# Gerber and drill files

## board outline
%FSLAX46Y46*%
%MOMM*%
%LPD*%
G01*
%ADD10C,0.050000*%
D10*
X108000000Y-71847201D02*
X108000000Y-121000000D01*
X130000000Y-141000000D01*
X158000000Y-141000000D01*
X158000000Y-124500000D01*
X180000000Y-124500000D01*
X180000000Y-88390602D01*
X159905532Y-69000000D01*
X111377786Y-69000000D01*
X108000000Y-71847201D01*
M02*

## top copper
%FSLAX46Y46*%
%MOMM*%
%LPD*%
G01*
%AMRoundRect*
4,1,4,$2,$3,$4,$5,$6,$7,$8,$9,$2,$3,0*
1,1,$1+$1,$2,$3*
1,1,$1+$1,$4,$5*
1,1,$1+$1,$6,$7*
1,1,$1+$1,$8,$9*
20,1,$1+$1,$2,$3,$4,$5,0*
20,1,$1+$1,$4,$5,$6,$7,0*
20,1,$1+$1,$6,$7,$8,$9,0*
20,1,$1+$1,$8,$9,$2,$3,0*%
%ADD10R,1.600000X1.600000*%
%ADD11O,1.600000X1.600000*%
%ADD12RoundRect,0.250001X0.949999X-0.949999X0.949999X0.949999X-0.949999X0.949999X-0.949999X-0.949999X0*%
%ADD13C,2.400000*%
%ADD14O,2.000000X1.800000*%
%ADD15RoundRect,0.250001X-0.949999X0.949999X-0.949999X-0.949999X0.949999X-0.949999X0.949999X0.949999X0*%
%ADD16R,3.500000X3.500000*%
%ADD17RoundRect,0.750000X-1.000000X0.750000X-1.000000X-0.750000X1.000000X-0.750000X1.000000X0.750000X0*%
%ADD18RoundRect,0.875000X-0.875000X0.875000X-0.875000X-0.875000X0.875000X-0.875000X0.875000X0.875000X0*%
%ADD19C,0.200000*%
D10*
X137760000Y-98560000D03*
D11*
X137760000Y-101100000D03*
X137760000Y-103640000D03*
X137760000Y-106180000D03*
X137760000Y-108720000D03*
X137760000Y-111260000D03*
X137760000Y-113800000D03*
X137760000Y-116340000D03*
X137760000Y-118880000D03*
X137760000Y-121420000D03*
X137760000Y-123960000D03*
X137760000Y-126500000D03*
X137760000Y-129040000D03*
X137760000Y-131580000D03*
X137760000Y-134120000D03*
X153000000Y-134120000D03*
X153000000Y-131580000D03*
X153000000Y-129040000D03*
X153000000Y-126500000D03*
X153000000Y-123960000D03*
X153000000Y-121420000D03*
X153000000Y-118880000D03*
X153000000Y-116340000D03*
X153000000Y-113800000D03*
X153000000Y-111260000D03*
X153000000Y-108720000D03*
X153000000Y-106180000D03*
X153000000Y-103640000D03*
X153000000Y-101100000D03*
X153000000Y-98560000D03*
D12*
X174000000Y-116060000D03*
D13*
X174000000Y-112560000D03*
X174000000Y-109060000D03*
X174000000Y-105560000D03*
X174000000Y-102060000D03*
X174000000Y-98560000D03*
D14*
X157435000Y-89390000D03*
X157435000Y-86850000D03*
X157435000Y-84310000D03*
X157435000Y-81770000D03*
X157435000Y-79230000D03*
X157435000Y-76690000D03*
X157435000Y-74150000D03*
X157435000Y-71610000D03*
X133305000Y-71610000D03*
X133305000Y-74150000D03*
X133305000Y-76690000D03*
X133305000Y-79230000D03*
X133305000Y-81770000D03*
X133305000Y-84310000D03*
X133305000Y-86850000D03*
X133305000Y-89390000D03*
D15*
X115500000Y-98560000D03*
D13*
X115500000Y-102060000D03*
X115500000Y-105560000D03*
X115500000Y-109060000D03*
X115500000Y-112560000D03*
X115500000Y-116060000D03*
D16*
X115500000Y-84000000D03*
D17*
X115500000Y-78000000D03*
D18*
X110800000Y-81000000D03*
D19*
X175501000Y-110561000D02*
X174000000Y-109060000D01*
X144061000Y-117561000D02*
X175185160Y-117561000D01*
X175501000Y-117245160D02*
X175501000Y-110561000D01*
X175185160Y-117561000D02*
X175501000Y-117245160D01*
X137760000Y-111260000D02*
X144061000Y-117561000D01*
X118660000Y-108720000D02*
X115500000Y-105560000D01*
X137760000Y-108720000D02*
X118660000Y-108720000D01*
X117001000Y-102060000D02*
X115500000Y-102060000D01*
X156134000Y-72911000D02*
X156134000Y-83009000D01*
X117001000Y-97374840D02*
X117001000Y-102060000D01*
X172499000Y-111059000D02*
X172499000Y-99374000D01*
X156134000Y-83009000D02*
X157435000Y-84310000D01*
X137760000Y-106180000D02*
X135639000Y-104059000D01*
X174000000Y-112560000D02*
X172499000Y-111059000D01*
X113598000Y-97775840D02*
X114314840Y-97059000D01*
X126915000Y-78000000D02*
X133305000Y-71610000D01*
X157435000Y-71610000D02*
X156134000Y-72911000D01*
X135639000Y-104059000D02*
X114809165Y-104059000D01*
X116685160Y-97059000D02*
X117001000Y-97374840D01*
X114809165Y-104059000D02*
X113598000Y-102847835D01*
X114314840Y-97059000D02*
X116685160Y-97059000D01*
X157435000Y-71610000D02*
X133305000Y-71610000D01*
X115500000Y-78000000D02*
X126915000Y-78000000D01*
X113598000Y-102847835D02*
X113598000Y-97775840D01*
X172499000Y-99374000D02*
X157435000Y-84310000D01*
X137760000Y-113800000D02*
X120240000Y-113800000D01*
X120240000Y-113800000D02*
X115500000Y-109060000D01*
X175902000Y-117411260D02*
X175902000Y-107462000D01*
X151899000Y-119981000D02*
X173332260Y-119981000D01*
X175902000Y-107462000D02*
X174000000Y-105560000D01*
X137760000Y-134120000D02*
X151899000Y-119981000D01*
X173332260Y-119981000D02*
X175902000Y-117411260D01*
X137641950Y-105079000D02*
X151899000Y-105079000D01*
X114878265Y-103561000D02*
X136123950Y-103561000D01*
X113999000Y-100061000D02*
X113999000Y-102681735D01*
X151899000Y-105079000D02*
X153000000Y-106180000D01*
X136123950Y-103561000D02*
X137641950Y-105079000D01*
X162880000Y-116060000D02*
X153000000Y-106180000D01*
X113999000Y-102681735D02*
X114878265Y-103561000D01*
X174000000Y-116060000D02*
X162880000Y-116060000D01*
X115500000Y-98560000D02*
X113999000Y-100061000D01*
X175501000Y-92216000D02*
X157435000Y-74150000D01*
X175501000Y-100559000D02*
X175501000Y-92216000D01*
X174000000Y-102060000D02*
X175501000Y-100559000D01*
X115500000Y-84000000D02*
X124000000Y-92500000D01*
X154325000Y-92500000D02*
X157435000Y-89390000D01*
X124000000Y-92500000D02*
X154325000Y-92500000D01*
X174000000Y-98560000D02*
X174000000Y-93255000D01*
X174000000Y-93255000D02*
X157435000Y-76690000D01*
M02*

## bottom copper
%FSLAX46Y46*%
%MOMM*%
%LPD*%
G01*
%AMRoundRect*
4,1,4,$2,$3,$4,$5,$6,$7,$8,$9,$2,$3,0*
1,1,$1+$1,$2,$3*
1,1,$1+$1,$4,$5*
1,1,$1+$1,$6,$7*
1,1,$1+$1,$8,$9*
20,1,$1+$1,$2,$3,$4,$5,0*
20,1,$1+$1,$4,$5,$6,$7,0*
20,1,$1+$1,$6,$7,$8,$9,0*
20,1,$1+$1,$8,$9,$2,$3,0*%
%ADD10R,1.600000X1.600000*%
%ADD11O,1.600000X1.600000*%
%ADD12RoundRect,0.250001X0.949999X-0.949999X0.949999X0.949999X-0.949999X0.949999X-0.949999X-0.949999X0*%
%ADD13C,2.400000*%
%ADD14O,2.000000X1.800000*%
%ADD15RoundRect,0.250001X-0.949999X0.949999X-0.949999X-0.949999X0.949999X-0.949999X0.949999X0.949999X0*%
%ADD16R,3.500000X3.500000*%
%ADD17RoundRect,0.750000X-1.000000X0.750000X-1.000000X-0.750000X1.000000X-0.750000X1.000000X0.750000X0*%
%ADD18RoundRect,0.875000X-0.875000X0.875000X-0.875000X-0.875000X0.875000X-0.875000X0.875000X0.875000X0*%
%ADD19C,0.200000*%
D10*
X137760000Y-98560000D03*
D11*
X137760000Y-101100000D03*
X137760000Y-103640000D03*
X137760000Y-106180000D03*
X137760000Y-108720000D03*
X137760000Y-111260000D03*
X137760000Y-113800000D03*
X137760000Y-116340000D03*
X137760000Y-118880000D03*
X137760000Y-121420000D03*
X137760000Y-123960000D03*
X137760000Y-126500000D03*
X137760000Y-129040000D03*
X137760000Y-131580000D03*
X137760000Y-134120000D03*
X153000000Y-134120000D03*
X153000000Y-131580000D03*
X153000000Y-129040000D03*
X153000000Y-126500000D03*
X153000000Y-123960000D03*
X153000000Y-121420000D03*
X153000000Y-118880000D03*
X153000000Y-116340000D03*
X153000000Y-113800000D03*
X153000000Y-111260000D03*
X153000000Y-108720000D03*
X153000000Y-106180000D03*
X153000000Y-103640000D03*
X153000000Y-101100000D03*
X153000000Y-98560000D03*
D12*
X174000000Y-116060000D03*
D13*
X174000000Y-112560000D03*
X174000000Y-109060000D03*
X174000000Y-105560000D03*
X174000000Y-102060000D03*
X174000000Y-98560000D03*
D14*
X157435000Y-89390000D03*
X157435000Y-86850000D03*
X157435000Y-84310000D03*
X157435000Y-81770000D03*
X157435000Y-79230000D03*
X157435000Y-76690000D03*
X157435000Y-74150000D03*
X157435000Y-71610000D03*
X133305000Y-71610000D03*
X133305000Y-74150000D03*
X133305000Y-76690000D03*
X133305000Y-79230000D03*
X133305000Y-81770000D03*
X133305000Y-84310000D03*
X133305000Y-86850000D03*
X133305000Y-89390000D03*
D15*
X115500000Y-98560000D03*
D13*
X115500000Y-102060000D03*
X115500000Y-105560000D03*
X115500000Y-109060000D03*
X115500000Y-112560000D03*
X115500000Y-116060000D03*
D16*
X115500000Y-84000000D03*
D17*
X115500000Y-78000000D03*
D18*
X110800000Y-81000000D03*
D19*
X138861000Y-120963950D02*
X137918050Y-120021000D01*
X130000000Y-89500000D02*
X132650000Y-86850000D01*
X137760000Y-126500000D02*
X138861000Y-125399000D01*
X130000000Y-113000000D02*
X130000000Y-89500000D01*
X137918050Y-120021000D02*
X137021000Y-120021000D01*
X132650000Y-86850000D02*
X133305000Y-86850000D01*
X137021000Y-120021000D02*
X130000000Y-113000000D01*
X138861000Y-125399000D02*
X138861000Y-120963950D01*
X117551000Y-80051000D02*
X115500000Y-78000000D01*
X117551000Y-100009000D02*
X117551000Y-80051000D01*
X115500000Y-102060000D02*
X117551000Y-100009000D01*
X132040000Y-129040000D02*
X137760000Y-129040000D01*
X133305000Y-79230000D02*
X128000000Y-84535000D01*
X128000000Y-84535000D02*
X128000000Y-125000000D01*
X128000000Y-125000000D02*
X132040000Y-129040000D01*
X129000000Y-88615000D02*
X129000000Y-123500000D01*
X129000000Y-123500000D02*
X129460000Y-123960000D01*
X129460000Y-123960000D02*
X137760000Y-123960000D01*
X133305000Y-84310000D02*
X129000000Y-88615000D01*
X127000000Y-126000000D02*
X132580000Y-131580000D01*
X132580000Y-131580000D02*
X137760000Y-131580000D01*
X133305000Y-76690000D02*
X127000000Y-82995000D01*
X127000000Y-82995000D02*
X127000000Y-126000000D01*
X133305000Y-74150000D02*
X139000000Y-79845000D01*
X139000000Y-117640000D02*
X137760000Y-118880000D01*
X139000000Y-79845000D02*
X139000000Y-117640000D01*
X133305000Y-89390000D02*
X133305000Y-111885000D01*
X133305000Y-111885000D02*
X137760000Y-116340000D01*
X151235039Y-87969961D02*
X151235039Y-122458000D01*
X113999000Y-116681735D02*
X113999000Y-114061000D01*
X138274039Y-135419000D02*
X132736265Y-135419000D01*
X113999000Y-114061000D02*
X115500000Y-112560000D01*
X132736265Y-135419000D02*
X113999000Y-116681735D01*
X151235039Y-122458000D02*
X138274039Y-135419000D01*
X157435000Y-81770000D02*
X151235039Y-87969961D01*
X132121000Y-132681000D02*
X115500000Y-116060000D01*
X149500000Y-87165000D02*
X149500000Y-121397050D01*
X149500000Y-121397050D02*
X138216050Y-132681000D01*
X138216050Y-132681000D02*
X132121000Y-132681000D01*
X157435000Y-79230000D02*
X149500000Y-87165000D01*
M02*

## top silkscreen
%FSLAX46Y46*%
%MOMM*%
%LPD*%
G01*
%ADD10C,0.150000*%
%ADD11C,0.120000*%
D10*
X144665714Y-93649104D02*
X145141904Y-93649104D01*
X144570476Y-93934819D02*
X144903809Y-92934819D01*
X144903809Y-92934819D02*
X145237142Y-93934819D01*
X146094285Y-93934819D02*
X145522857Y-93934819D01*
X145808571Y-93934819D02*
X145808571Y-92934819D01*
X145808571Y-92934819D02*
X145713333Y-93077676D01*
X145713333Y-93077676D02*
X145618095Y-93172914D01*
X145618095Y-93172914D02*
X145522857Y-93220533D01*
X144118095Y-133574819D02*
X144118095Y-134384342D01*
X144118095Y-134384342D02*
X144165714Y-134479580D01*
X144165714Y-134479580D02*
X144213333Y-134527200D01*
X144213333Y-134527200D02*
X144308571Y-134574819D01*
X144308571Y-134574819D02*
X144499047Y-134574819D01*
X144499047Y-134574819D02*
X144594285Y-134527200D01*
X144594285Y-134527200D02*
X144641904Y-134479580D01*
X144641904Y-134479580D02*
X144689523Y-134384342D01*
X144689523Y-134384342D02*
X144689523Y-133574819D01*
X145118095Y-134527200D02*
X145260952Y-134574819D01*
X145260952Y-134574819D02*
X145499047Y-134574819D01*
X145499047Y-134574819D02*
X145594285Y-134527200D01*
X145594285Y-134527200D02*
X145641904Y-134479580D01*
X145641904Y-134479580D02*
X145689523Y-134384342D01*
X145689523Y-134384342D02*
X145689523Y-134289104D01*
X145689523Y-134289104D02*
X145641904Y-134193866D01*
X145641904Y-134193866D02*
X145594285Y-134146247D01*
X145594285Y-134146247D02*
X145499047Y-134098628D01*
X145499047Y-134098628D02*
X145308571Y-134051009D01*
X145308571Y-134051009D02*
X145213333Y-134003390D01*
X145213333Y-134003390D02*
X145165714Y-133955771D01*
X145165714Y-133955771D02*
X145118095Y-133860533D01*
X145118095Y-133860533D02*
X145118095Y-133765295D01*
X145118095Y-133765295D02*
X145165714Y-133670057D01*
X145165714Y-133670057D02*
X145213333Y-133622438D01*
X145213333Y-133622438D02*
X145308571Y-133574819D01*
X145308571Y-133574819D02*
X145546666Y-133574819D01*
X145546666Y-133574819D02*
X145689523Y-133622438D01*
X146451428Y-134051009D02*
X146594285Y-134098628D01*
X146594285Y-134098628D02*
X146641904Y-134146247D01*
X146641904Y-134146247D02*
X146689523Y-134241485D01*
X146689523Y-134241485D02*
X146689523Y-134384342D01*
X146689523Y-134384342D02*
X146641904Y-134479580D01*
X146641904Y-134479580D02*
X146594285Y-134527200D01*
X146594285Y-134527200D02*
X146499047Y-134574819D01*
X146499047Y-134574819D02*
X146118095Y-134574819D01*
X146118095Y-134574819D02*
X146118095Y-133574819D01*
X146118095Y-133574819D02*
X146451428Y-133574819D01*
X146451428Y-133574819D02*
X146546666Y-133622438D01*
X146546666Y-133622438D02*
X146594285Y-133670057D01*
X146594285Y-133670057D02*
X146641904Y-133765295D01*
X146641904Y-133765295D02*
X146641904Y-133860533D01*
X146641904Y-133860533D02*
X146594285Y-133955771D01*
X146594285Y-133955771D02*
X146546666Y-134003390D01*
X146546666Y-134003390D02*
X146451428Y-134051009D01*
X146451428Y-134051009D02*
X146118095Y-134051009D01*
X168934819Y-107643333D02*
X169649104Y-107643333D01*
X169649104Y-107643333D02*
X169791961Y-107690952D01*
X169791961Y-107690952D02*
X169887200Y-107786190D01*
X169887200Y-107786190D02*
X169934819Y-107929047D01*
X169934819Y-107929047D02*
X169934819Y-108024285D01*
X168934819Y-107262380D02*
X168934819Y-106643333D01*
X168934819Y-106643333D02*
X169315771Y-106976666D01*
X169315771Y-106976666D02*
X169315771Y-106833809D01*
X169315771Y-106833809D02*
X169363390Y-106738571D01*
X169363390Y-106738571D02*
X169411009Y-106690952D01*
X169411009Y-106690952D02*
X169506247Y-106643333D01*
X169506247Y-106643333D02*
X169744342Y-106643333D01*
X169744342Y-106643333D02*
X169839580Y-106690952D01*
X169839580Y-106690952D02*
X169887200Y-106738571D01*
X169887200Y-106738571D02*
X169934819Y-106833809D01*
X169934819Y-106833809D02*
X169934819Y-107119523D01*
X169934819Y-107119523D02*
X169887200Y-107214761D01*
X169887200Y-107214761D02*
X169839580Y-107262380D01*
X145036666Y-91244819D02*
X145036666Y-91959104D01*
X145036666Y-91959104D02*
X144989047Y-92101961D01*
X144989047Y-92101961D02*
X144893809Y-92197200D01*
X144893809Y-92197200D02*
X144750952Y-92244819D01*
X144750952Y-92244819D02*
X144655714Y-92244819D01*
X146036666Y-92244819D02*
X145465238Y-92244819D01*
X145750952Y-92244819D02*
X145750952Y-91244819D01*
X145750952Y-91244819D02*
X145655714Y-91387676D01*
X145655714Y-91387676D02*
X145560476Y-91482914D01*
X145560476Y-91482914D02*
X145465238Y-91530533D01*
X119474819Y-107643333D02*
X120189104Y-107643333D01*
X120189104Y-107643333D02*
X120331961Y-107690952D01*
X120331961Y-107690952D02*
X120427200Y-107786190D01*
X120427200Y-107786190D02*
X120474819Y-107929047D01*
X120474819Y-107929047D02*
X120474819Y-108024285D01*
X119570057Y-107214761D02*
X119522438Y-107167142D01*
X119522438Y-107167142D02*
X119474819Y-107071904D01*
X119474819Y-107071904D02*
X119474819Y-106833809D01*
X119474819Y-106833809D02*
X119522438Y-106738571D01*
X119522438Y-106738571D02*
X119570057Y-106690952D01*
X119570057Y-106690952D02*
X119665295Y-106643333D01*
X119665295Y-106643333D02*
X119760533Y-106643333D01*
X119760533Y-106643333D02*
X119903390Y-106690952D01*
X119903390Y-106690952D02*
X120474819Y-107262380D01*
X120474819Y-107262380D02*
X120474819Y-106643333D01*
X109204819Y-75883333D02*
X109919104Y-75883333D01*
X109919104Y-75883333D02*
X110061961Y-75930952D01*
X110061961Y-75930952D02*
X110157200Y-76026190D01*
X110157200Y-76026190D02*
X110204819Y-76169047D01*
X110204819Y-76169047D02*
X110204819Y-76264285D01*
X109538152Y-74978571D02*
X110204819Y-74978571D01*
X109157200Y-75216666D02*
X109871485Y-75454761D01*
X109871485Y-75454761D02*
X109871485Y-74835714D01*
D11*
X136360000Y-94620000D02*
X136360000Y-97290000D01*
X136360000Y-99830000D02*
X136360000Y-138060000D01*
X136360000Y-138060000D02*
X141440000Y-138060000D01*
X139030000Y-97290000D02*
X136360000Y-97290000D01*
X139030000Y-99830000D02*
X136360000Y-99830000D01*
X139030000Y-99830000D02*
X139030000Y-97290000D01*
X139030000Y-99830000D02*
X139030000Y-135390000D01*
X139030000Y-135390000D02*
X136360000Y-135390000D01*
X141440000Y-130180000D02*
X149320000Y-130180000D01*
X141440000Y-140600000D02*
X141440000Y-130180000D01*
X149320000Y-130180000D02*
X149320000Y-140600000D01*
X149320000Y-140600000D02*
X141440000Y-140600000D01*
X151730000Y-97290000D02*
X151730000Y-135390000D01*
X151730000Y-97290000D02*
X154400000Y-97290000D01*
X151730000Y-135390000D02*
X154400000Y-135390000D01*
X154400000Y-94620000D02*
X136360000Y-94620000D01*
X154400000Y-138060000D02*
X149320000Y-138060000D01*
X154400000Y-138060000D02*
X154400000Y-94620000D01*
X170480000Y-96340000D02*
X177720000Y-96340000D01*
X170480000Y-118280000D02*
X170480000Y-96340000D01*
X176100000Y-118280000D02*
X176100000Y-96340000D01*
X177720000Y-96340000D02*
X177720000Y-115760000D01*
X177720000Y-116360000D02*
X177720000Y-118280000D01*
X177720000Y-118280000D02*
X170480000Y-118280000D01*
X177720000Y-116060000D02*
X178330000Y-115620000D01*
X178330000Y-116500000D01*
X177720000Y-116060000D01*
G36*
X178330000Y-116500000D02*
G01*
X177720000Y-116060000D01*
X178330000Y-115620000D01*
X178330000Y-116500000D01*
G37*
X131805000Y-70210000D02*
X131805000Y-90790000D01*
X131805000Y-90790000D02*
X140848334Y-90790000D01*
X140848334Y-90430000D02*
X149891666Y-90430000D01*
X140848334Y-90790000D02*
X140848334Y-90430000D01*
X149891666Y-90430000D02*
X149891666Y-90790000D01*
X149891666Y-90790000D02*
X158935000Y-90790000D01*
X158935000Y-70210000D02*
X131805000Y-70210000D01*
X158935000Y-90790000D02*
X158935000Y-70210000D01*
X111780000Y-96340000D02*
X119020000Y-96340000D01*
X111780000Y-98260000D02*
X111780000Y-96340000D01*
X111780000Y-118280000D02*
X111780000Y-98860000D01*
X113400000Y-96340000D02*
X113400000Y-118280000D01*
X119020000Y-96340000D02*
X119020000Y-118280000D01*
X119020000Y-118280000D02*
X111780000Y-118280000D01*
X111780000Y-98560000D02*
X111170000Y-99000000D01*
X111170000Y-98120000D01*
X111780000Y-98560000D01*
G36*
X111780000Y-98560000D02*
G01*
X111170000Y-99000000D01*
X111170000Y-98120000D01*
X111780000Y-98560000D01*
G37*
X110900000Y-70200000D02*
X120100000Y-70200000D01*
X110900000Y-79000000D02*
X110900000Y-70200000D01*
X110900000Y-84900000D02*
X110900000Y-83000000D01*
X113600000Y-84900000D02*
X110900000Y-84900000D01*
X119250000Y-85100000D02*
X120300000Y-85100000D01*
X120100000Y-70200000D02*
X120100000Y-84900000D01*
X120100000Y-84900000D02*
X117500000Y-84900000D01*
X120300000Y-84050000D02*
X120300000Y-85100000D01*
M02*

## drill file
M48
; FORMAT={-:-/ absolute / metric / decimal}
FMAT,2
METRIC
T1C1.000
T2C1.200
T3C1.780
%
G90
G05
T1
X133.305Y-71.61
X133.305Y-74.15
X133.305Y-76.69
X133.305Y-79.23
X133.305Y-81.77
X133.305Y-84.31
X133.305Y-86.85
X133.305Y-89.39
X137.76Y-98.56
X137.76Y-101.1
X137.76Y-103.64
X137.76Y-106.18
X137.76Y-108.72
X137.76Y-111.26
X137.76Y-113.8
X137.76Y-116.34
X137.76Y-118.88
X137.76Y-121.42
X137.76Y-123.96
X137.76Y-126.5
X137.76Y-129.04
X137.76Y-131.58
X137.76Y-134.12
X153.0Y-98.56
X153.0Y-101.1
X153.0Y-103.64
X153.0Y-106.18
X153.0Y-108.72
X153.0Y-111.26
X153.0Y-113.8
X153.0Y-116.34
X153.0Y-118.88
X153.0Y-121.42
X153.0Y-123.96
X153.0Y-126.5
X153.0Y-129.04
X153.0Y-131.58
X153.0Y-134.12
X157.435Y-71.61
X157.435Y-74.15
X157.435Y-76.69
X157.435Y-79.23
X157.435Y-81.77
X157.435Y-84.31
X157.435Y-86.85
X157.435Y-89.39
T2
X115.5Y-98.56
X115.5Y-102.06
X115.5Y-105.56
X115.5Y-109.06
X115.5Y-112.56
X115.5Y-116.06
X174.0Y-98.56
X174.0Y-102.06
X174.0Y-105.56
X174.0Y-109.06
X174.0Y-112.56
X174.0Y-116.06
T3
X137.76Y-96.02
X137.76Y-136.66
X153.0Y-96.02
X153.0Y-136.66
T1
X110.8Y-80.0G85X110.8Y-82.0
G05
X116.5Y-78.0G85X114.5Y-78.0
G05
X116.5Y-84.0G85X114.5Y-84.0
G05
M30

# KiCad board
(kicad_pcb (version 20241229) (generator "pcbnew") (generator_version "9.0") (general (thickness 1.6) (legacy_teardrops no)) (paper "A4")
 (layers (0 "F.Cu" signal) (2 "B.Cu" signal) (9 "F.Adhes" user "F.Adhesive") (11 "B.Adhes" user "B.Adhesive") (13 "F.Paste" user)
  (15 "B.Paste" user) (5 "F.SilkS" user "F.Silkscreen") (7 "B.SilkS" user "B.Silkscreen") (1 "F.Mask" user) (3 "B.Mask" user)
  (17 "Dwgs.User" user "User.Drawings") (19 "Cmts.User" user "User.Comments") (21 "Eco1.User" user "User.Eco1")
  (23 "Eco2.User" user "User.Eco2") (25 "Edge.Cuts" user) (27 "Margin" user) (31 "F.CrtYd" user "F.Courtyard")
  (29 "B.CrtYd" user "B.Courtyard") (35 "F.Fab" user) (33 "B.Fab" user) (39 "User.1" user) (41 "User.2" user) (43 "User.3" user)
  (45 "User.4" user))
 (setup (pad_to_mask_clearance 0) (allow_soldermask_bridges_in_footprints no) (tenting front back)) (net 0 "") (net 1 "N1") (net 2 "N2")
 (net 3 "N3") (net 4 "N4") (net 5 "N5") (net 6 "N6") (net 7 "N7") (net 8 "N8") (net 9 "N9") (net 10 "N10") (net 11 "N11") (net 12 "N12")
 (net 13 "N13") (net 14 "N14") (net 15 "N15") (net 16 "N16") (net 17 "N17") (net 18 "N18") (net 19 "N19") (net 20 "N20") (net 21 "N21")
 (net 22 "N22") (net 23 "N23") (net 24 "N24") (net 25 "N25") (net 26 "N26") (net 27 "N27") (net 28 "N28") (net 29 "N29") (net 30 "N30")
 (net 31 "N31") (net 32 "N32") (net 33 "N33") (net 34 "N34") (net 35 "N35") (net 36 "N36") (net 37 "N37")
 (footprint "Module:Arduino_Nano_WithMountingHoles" (layer "F.Cu") (at 137.76 98.56)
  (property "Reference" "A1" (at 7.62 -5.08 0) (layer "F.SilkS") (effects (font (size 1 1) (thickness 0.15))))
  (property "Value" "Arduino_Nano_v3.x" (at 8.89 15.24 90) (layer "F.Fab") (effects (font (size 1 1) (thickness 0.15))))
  (fp_line (start -1.4 -3.94) (end -1.4 -1.27) (stroke (width 0.12) (type solid)) (layer "F.SilkS"))
  (fp_line (start -1.4 1.27) (end -1.4 39.5) (stroke (width 0.12) (type solid)) (layer "F.SilkS"))
  (fp_line (start -1.4 39.5) (end 3.68 39.5) (stroke (width 0.12) (type solid)) (layer "F.SilkS"))
  (fp_line (start 1.27 -1.27) (end -1.4 -1.27) (stroke (width 0.12) (type solid)) (layer "F.SilkS"))
  (fp_line (start 1.27 1.27) (end -1.4 1.27) (stroke (width 0.12) (type solid)) (layer "F.SilkS"))
  (fp_line (start 1.27 1.27) (end 1.27 -1.27) (stroke (width 0.12) (type solid)) (layer "F.SilkS"))
  (fp_line (start 1.27 1.27) (end 1.27 36.83) (stroke (width 0.12) (type solid)) (layer "F.SilkS"))
  (fp_line (start 1.27 36.83) (end -1.4 36.83) (stroke (width 0.12) (type solid)) (layer "F.SilkS"))
  (fp_line (start 3.68 31.62) (end 11.56 31.62) (stroke (width 0.12) (type solid)) (layer "F.SilkS"))
  (fp_line (start 3.68 42.04) (end 3.68 31.62) (stroke (width 0.12) (type solid)) (layer "F.SilkS"))
  (fp_line (start 11.56 31.62) (end 11.56 42.04) (stroke (width 0.12) (type solid)) (layer "F.SilkS"))
  (fp_line (start 11.56 42.04) (end 3.68 42.04) (stroke (width 0.12) (type solid)) (layer "F.SilkS"))
  (fp_line (start 13.97 -1.27) (end 13.97 36.83) (stroke (width 0.12) (type solid)) (layer "F.SilkS"))
  (fp_line (start 13.97 -1.27) (end 16.64 -1.27) (stroke (width 0.12) (type solid)) (layer "F.SilkS"))
  (fp_line (start 13.97 36.83) (end 16.64 36.83) (stroke (width 0.12) (type solid)) (layer "F.SilkS"))
  (fp_line (start 16.64 -3.94) (end -1.4 -3.94) (stroke (width 0.12) (type solid)) (layer "F.SilkS"))
  (fp_line (start 16.64 39.5) (end 11.56 39.5) (stroke (width 0.12) (type solid)) (layer "F.SilkS"))
  (fp_line (start 16.64 39.5) (end 16.64 -3.94) (stroke (width 0.12) (type solid)) (layer "F.SilkS"))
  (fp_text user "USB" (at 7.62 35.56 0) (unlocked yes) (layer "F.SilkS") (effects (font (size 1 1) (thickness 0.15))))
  (pad "" np_thru_hole circle (at 0 -2.54) (size 1.78 1.78) (drill 1.78) (layers "*.Cu" "*.Mask"))
  (pad "" np_thru_hole circle (at 0 38.1) (size 1.78 1.78) (drill 1.78) (layers "*.Cu" "*.Mask"))
  (pad "" np_thru_hole circle (at 15.24 -2.54) (size 1.78 1.78) (drill 1.78) (layers "*.Cu" "*.Mask"))
  (pad "" np_thru_hole circle (at 15.24 38.1) (size 1.78 1.78) (drill 1.78) (layers "*.Cu" "*.Mask"))
  (pad "1" thru_hole rect (at 0 0) (size 1.6 1.6) (drill 1) (layers "*.Cu" "*.Mask") (remove_unused_layers no) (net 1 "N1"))
  (pad "2" thru_hole oval (at 0 2.54) (size 1.6 1.6) (drill 1) (layers "*.Cu" "*.Mask") (remove_unused_layers no) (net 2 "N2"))
  (pad "3" thru_hole oval (at 0 5.08) (size 1.6 1.6) (drill 1) (layers "*.Cu" "*.Mask") (remove_unused_layers no) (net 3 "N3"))
  (pad "4" thru_hole oval (at 0 7.62) (size 1.6 1.6) (drill 1) (layers "*.Cu" "*.Mask") (remove_unused_layers no) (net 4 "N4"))
  (pad "5" thru_hole oval (at 0 10.16) (size 1.6 1.6) (drill 1) (layers "*.Cu" "*.Mask") (remove_unused_layers no) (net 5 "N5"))
  (pad "6" thru_hole oval (at 0 12.7) (size 1.6 1.6) (drill 1) (layers "*.Cu" "*.Mask") (remove_unused_layers no) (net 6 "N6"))
  (pad "7" thru_hole oval (at 0 15.24) (size 1.6 1.6) (drill 1) (layers "*.Cu" "*.Mask") (remove_unused_layers no) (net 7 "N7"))
  (pad "8" thru_hole oval (at 0 17.78) (size 1.6 1.6) (drill 1) (layers "*.Cu" "*.Mask") (remove_unused_layers no) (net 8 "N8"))
  (pad "9" thru_hole oval (at 0 20.32) (size 1.6 1.6) (drill 1) (layers "*.Cu" "*.Mask") (remove_unused_layers no) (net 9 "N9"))
  (pad "10" thru_hole oval (at 0 22.86) (size 1.6 1.6) (drill 1) (layers "*.Cu" "*.Mask") (remove_unused_layers no) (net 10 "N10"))
  (pad "11" thru_hole oval (at 0 25.4) (size 1.6 1.6) (drill 1) (layers "*.Cu" "*.Mask") (remove_unused_layers no) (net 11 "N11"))
  (pad "12" thru_hole oval (at 0 27.94) (size 1.6 1.6) (drill 1) (layers "*.Cu" "*.Mask") (remove_unused_layers no) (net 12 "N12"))
  (pad "13" thru_hole oval (at 0 30.48) (size 1.6 1.6) (drill 1) (layers "*.Cu" "*.Mask") (remove_unused_layers no) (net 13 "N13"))
  (pad "14" thru_hole oval (at 0 33.02) (size 1.6 1.6) (drill 1) (layers "*.Cu" "*.Mask") (remove_unused_layers no) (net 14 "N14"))
  (pad "15" thru_hole oval (at 0 35.56) (size 1.6 1.6) (drill 1) (layers "*.Cu" "*.Mask") (remove_unused_layers no) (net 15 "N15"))
  (pad "16" thru_hole oval (at 15.24 35.56) (size 1.6 1.6) (drill 1) (layers "*.Cu" "*.Mask") (remove_unused_layers no) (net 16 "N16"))
  (pad "17" thru_hole oval (at 15.24 33.02) (size 1.6 1.6) (drill 1) (layers "*.Cu" "*.Mask") (remove_unused_layers no) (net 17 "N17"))
  (pad "18" thru_hole oval (at 15.24 30.48) (size 1.6 1.6) (drill 1) (layers "*.Cu" "*.Mask") (remove_unused_layers no) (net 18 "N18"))
  (pad "19" thru_hole oval (at 15.24 27.94) (size 1.6 1.6) (drill 1) (layers "*.Cu" "*.Mask") (remove_unused_layers no) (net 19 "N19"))
  (pad "20" thru_hole oval (at 15.24 25.4) (size 1.6 1.6) (drill 1) (layers "*.Cu" "*.Mask") (remove_unused_layers no) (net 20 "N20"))
  (pad "21" thru_hole oval (at 15.24 22.86) (size 1.6 1.6) (drill 1) (layers "*.Cu" "*.Mask") (remove_unused_layers no) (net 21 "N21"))
  (pad "22" thru_hole oval (at 15.24 20.32) (size 1.6 1.6) (drill 1) (layers "*.Cu" "*.Mask") (remove_unused_layers no) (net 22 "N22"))
  (pad "23" thru_hole oval (at 15.24 17.78) (size 1.6 1.6) (drill 1) (layers "*.Cu" "*.Mask") (remove_unused_layers no) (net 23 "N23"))
  (pad "24" thru_hole oval (at 15.24 15.24) (size 1.6 1.6) (drill 1) (layers "*.Cu" "*.Mask") (remove_unused_layers no) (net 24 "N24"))
  (pad "25" thru_hole oval (at 15.24 12.7) (size 1.6 1.6) (drill 1) (layers "*.Cu" "*.Mask") (remove_unused_layers no) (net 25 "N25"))
  (pad "26" thru_hole oval (at 15.24 10.16) (size 1.6 1.6) (drill 1) (layers "*.Cu" "*.Mask") (remove_unused_layers no) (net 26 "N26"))
  (pad "27" thru_hole oval (at 15.24 7.62) (size 1.6 1.6) (drill 1) (layers "*.Cu" "*.Mask") (remove_unused_layers no) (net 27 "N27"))
  (pad "28" thru_hole oval (at 15.24 5.08) (size 1.6 1.6) (drill 1) (layers "*.Cu" "*.Mask") (remove_unused_layers no) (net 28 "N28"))
  (pad "29" thru_hole oval (at 15.24 2.54) (size 1.6 1.6) (drill 1) (layers "*.Cu" "*.Mask") (remove_unused_layers no) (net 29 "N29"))
  (pad "30" thru_hole oval (at 15.24 0) (size 1.6 1.6) (drill 1) (layers "*.Cu" "*.Mask") (remove_unused_layers no) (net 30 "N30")))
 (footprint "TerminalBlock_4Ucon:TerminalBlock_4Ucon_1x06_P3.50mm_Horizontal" (layer "F.Cu") (at 174 116.06 90)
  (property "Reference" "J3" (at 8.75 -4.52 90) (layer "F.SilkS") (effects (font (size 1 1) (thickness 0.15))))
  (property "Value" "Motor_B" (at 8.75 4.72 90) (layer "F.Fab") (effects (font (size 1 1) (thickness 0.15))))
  (fp_line (start 19.72 -3.52) (end 19.72 3.72) (stroke (width 0.12) (type solid)) (layer "F.SilkS"))
  (fp_line (start -2.22 -3.52) (end 19.72 -3.52) (stroke (width 0.12) (type solid)) (layer "F.SilkS"))
  (fp_line (start -2.22 2.1) (end 19.72 2.1) (stroke (width 0.12) (type solid)) (layer "F.SilkS"))
  (fp_line (start 19.72 3.72) (end 0.3 3.72) (stroke (width 0.12) (type solid)) (layer "F.SilkS"))
  (fp_line (start -0.3 3.72) (end -2.22 3.72) (stroke (width 0.12) (type solid)) (layer "F.SilkS"))
  (fp_line (start -2.22 3.72) (end -2.22 -3.52) (stroke (width 0.12) (type solid)) (layer "F.SilkS"))
  (fp_poly (pts (xy 0 3.72) (xy 0.44 4.33) (xy -0.44 4.33)) (stroke (width 0.12) (type solid)) (fill yes) (layer "F.SilkS"))
  (pad "1" thru_hole roundrect (at 0 0 90) (size 2.4 2.4) (drill 1.2) (layers "*.Cu" "*.Mask") (remove_unused_layers no)
   (roundrect_rratio 0.104167) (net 27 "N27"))
  (pad "2" thru_hole circle (at 3.5 0 90) (size 2.4 2.4) (drill 1.2) (layers "*.Cu" "*.Mask") (remove_unused_layers no) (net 4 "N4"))
  (pad "3" thru_hole circle (at 7 0 90) (size 2.4 2.4) (drill 1.2) (layers "*.Cu" "*.Mask") (remove_unused_layers no) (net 6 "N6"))
  (pad "4" thru_hole circle (at 10.5 0 90) (size 2.4 2.4) (drill 1.2) (layers "*.Cu" "*.Mask") (remove_unused_layers no) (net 15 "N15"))
  (pad "5" thru_hole circle (at 14 0 90) (size 2.4 2.4) (drill 1.2) (layers "*.Cu" "*.Mask") (remove_unused_layers no) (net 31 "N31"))
  (pad "6" thru_hole circle (at 17.5 0 90) (size 2.4 2.4) (drill 1.2) (layers "*.Cu" "*.Mask") (remove_unused_layers no) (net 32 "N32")))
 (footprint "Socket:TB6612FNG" (layer "F.Cu") (at 145.37 80.5 90)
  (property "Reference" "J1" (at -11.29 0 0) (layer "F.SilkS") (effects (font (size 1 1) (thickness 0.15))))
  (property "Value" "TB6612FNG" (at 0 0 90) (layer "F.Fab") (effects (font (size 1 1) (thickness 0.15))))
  (fp_line (start 10.29 -13.565) (end -10.29 -13.565) (stroke (width 0.12) (type default)) (layer "F.SilkS"))
  (fp_line (start -10.29 -13.565) (end -10.29 -4.521666) (stroke (width 0.12) (type default)) (layer "F.SilkS"))
  (fp_line (start -9.93 -4.521666) (end -9.93 4.521666) (stroke (width 0.12) (type default)) (layer "F.SilkS"))
  (fp_line (start -10.29 -4.521666) (end -9.93 -4.521666) (stroke (width 0.12) (type default)) (layer "F.SilkS"))
  (fp_line (start -9.93 4.521666) (end -10.29 4.521666) (stroke (width 0.12) (type default)) (layer "F.SilkS"))
  (fp_line (start -10.29 4.521666) (end -10.29 13.565) (stroke (width 0.12) (type default)) (layer "F.SilkS"))
  (fp_line (start 10.29 13.565) (end 10.29 -13.565) (stroke (width 0.12) (type default)) (layer "F.SilkS"))
  (fp_line (start -10.29 13.565) (end 10.29 13.565) (stroke (width 0.12) (type default)) (layer "F.SilkS"))
  (pad "1" thru_hole oval (at -8.89 12.065 90) (size 1.8 2) (drill 1) (layers "*.Cu" "*.Mask") (remove_unused_layers no) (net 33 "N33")
   (thermal_bridge_angle 45))
  (pad "2" thru_hole oval (at -6.35 12.065 90) (size 1.8 2) (drill 1) (layers "*.Cu" "*.Mask") (remove_unused_layers no) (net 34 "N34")
   (thermal_bridge_angle 45))
  (pad "3" thru_hole oval (at -3.81 12.065 90) (size 1.8 2) (drill 1) (layers "*.Cu" "*.Mask") (remove_unused_layers no) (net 4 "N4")
   (thermal_bridge_angle 45))
  (pad "4" thru_hole oval (at -1.27 12.065 90) (size 1.8 2) (drill 1) (layers "*.Cu" "*.Mask") (remove_unused_layers no) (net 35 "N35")
   (thermal_bridge_angle 45))
  (pad "5" thru_hole oval (at 1.27 12.065 90) (size 1.8 2) (drill 1) (layers "*.Cu" "*.Mask") (remove_unused_layers no) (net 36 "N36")
   (thermal_bridge_angle 45))
  (pad "6" thru_hole oval (at 3.81 12.065 90) (size 1.8 2) (drill 1) (layers "*.Cu" "*.Mask") (remove_unused_layers no) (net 32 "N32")
   (thermal_bridge_angle 45))
  (pad "7" thru_hole oval (at 6.35 12.065 90) (size 1.8 2) (drill 1) (layers "*.Cu" "*.Mask") (remove_unused_layers no) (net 31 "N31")
   (thermal_bridge_angle 45))
  (pad "8" thru_hole oval (at 8.89 12.065 90) (size 1.8 2) (drill 1) (layers "*.Cu" "*.Mask") (remove_unused_layers no) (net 4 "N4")
   (thermal_bridge_angle 45))
  (pad "9" thru_hole oval (at 8.89 -12.065 90) (size 1.8 2) (drill 1) (layers "*.Cu" "*.Mask") (remove_unused_layers no) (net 4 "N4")
   (thermal_bridge_angle 45))
  (pad "10" thru_hole oval (at 6.35 -12.065 90) (size 1.8 2) (drill 1) (layers "*.Cu" "*.Mask") (remove_unused_layers no) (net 9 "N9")
   (thermal_bridge_angle 45))
  (pad "11" thru_hole oval (at 3.81 -12.065 90) (size 1.8 2) (drill 1) (layers "*.Cu" "*.Mask") (remove_unused_layers no) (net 14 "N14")
   (thermal_bridge_angle 45))
  (pad "12" thru_hole oval (at 1.27 -12.065 90) (size 1.8 2) (drill 1) (layers "*.Cu" "*.Mask") (remove_unused_layers no) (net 13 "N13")
   (thermal_bridge_angle 45))
  (pad "13" thru_hole oval (at -1.27 -12.065 90) (size 1.8 2) (drill 1) (layers "*.Cu" "*.Mask") (remove_unused_layers no) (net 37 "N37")
   (thermal_bridge_angle 45))
  (pad "14" thru_hole oval (at -3.81 -12.065 90) (size 1.8 2) (drill 1) (layers "*.Cu" "*.Mask") (remove_unused_layers no) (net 11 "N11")
   (thermal_bridge_angle 45))
  (pad "15" thru_hole oval (at -6.35 -12.065 90) (size 1.8 2) (drill 1) (layers "*.Cu" "*.Mask") (remove_unused_layers no) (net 12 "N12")
   (thermal_bridge_angle 45))
  (pad "16" thru_hole oval (at -8.89 -12.065 90) (size 1.8 2) (drill 1) (layers "*.Cu" "*.Mask") (remove_unused_layers no) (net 8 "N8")
   (thermal_bridge_angle 45)))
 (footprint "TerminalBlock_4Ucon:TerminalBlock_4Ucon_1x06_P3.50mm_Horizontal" (layer "F.Cu") (at 115.5 98.56 -90)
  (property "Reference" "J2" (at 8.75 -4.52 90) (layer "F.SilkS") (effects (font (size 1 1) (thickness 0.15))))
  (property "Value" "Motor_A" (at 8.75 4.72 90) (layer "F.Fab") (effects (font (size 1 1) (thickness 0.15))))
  (fp_line (start -2.22 3.72) (end -2.22 -3.52) (stroke (width 0.12) (type solid)) (layer "F.SilkS"))
  (fp_line (start -0.3 3.72) (end -2.22 3.72) (stroke (width 0.12) (type solid)) (layer "F.SilkS"))
  (fp_line (start 19.72 3.72) (end 0.3 3.72) (stroke (width 0.12) (type solid)) (layer "F.SilkS"))
  (fp_line (start -2.22 2.1) (end 19.72 2.1) (stroke (width 0.12) (type solid)) (layer "F.SilkS"))
  (fp_line (start -2.22 -3.52) (end 19.72 -3.52) (stroke (width 0.12) (type solid)) (layer "F.SilkS"))
  (fp_line (start 19.72 -3.52) (end 19.72 3.72) (stroke (width 0.12) (type solid)) (layer "F.SilkS"))
  (fp_poly (pts (xy 0 3.72) (xy 0.44 4.33) (xy -0.44 4.33)) (stroke (width 0.12) (type solid)) (fill yes) (layer "F.SilkS"))
  (pad "1" thru_hole roundrect (at 0 0 270) (size 2.4 2.4) (drill 1.2) (layers "*.Cu" "*.Mask") (remove_unused_layers no)
   (roundrect_rratio 0.104167) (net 27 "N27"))
  (pad "2" thru_hole circle (at 3.5 0 270) (size 2.4 2.4) (drill 1.2) (layers "*.Cu" "*.Mask") (remove_unused_layers no) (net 4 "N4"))
  (pad "3" thru_hole circle (at 7 0 270) (size 2.4 2.4) (drill 1.2) (layers "*.Cu" "*.Mask") (remove_unused_layers no) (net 5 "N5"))
  (pad "4" thru_hole circle (at 10.5 0 270) (size 2.4 2.4) (drill 1.2) (layers "*.Cu" "*.Mask") (remove_unused_layers no) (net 7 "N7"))
  (pad "5" thru_hole circle (at 14 0 270) (size 2.4 2.4) (drill 1.2) (layers "*.Cu" "*.Mask") (remove_unused_layers no) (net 35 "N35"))
  (pad "6" thru_hole circle (at 17.5 0 270) (size 2.4 2.4) (drill 1.2) (layers "*.Cu" "*.Mask") (remove_unused_layers no) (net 36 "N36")))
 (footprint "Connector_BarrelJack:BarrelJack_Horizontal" (layer "F.Cu") (at 115.5 84 -90)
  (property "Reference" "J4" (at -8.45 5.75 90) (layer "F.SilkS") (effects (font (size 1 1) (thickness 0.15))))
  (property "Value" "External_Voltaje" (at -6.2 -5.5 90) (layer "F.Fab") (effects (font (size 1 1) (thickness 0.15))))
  (fp_line (start -13.8 4.6) (end -13.8 -4.6) (stroke (width 0.12) (type solid)) (layer "F.SilkS"))
  (fp_line (start -5 4.6) (end -13.8 4.6) (stroke (width 0.12) (type solid)) (layer "F.SilkS"))
  (fp_line (start 0.9 4.6) (end -1 4.6) (stroke (width 0.12) (type solid)) (layer "F.SilkS"))
  (fp_line (start 0.9 1.9) (end 0.9 4.6) (stroke (width 0.12) (type solid)) (layer "F.SilkS"))
  (fp_line (start 1.1 -3.75) (end 1.1 -4.8) (stroke (width 0.12) (type solid)) (layer "F.SilkS"))
  (fp_line (start -13.8 -4.6) (end 0.9 -4.6) (stroke (width 0.12) (type solid)) (layer "F.SilkS"))
  (fp_line (start 0.9 -4.6) (end 0.9 -2) (stroke (width 0.12) (type solid)) (layer "F.SilkS"))
  (fp_line (start 0.05 -4.8) (end 1.1 -4.8) (stroke (width 0.12) (type solid)) (layer "F.SilkS"))
  (pad "1" thru_hole rect (at 0 0 270) (size 3.5 3.5) (drill oval 1 3) (layers "*.Cu" "*.Mask") (remove_unused_layers no) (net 33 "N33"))
  (pad "2" thru_hole roundrect (at -6 0 270) (size 3 3.5) (drill oval 1 3) (layers "*.Cu" "*.Mask") (remove_unused_layers no)
   (roundrect_rratio 0.25) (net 4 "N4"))
  (pad "3" thru_hole roundrect (at -3 4.7 270) (size 3.5 3.5) (drill oval 3 1) (layers "*.Cu" "*.Mask") (remove_unused_layers no)
   (roundrect_rratio 0.25)))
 (gr_poly
  (pts (xy 108 71.847201) (xy 108 121) (xy 130 141) (xy 158 141) (xy 158 124.5) (xy 180 124.5) (xy 180 88.390602) (xy 159.905532 69)
   (xy 111.377786 69))
  (stroke (width 0.05) (type solid)) (fill no) (layer "Edge.Cuts"))
 (segment (start 175.501 110.561) (end 174 109.06) (width 0.2) (layer "F.Cu") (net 6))
 (segment (start 144.061 117.561) (end 175.18516 117.561) (width 0.2) (layer "F.Cu") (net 6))
 (segment (start 175.501 117.24516) (end 175.501 110.561) (width 0.2) (layer "F.Cu") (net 6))
 (segment (start 175.18516 117.561) (end 175.501 117.24516) (width 0.2) (layer "F.Cu") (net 6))
 (segment (start 137.76 111.26) (end 144.061 117.561) (width 0.2) (layer "F.Cu") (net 6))
 (segment (start 118.66 108.72) (end 115.5 105.56) (width 0.2) (layer "F.Cu") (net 5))
 (segment (start 137.76 108.72) (end 118.66 108.72) (width 0.2) (layer "F.Cu") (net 5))
 (segment (start 138.861 120.96395) (end 137.91805 120.021) (width 0.2) (layer "B.Cu") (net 12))
 (segment (start 130 89.5) (end 132.65 86.85) (width 0.2) (layer "B.Cu") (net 12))
 (segment (start 137.76 126.5) (end 138.861 125.399) (width 0.2) (layer "B.Cu") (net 12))
 (segment (start 130 113) (end 130 89.5) (width 0.2) (layer "B.Cu") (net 12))
 (segment (start 137.91805 120.021) (end 137.021 120.021) (width 0.2) (layer "B.Cu") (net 12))
 (segment (start 132.65 86.85) (end 133.305 86.85) (width 0.2) (layer "B.Cu") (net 12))
 (segment (start 137.021 120.021) (end 130 113) (width 0.2) (layer "B.Cu") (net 12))
 (segment (start 138.861 125.399) (end 138.861 120.96395) (width 0.2) (layer "B.Cu") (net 12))
 (segment (start 117.001 102.06) (end 115.5 102.06) (width 0.2) (layer "F.Cu") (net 4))
 (segment (start 156.134 72.911) (end 156.134 83.009) (width 0.2) (layer "F.Cu") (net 4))
 (segment (start 117.001 97.37484) (end 117.001 102.06) (width 0.2) (layer "F.Cu") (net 4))
 (segment (start 172.499 111.059) (end 172.499 99.374) (width 0.2) (layer "F.Cu") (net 4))
 (segment (start 156.134 83.009) (end 157.435 84.31) (width 0.2) (layer "F.Cu") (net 4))
 (segment (start 137.76 106.18) (end 135.639 104.059) (width 0.2) (layer "F.Cu") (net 4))
 (segment (start 174 112.56) (end 172.499 111.059) (width 0.2) (layer "F.Cu") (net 4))
 (segment (start 113.598 97.77584) (end 114.31484 97.059) (width 0.2) (layer "F.Cu") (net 4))
 (segment (start 126.915 78) (end 133.305 71.61) (width 0.2) (layer "F.Cu") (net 4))
 (segment (start 157.435 71.61) (end 156.134 72.911) (width 0.2) (layer "F.Cu") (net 4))
 (segment (start 135.639 104.059) (end 114.809165 104.059) (width 0.2) (layer "F.Cu") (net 4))
 (segment (start 116.68516 97.059) (end 117.001 97.37484) (width 0.2) (layer "F.Cu") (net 4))
 (segment (start 114.809165 104.059) (end 113.598 102.847835) (width 0.2) (layer "F.Cu") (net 4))
 (segment (start 114.31484 97.059) (end 116.68516 97.059) (width 0.2) (layer "F.Cu") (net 4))
 (segment (start 157.435 71.61) (end 133.305 71.61) (width 0.2) (layer "F.Cu") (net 4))
 (segment (start 115.5 78) (end 126.915 78) (width 0.2) (layer "F.Cu") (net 4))
 (segment (start 113.598 102.847835) (end 113.598 97.77584) (width 0.2) (layer "F.Cu") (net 4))
 (segment (start 172.499 99.374) (end 157.435 84.31) (width 0.2) (layer "F.Cu") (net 4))
 (segment (start 117.551 80.051) (end 115.5 78) (width 0.2) (layer "B.Cu") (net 4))
 (segment (start 117.551 100.009) (end 117.551 80.051) (width 0.2) (layer "B.Cu") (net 4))
 (segment (start 115.5 102.06) (end 117.551 100.009) (width 0.2) (layer "B.Cu") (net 4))
 (segment (start 132.04 129.04) (end 137.76 129.04) (width 0.2) (layer "B.Cu") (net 13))
 (segment (start 133.305 79.23) (end 128 84.535) (width 0.2) (layer "B.Cu") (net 13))
 (segment (start 128 84.535) (end 128 125) (width 0.2) (layer "B.Cu") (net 13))
 (segment (start 128 125) (end 132.04 129.04) (width 0.2) (layer "B.Cu") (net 13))
 (segment (start 129 88.615) (end 129 123.5) (width 0.2) (layer "B.Cu") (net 11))
 (segment (start 129 123.5) (end 129.46 123.96) (width 0.2) (layer "B.Cu") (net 11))
 (segment (start 129.46 123.96) (end 137.76 123.96) (width 0.2) (layer "B.Cu") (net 11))
 (segment (start 133.305 84.31) (end 129 88.615) (width 0.2) (layer "B.Cu") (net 11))
 (segment (start 127 126) (end 132.58 131.58) (width 0.2) (layer "B.Cu") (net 14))
 (segment (start 132.58 131.58) (end 137.76 131.58) (width 0.2) (layer "B.Cu") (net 14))
 (segment (start 133.305 76.69) (end 127 82.995) (width 0.2) (layer "B.Cu") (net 14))
 (segment (start 127 82.995) (end 127 126) (width 0.2) (layer "B.Cu") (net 14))
 (segment (start 137.76 113.8) (end 120.24 113.8) (width 0.2) (layer "F.Cu") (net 7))
 (segment (start 120.24 113.8) (end 115.5 109.06) (width 0.2) (layer "F.Cu") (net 7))
 (segment (start 175.902 117.41126) (end 175.902 107.462) (width 0.2) (layer "F.Cu") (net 15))
 (segment (start 151.899 119.981) (end 173.33226 119.981) (width 0.2) (layer "F.Cu") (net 15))
 (segment (start 175.902 107.462) (end 174 105.56) (width 0.2) (layer "F.Cu") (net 15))
 (segment (start 137.76 134.12) (end 151.899 119.981) (width 0.2) (layer "F.Cu") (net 15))
 (segment (start 173.33226 119.981) (end 175.902 117.41126) (width 0.2) (layer "F.Cu") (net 15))
 (segment (start 137.64195 105.079) (end 151.899 105.079) (width 0.2) (layer "F.Cu") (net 27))
 (segment (start 114.878265 103.561) (end 136.12395 103.561) (width 0.2) (layer "F.Cu") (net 27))
 (segment (start 113.999 100.061) (end 113.999 102.681735) (width 0.2) (layer "F.Cu") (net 27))
 (segment (start 151.899 105.079) (end 153 106.18) (width 0.2) (layer "F.Cu") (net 27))
 (segment (start 136.12395 103.561) (end 137.64195 105.079) (width 0.2) (layer "F.Cu") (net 27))
 (segment (start 162.88 116.06) (end 153 106.18) (width 0.2) (layer "F.Cu") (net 27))
 (segment (start 113.999 102.681735) (end 114.878265 103.561) (width 0.2) (layer "F.Cu") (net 27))
 (segment (start 174 116.06) (end 162.88 116.06) (width 0.2) (layer "F.Cu") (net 27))
 (segment (start 115.5 98.56) (end 113.999 100.061) (width 0.2) (layer "F.Cu") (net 27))
 (segment (start 133.305 74.15) (end 139 79.845) (width 0.2) (layer "B.Cu") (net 9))
 (segment (start 139 117.64) (end 137.76 118.88) (width 0.2) (layer "B.Cu") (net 9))
 (segment (start 139 79.845) (end 139 117.64) (width 0.2) (layer "B.Cu") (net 9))
 (segment (start 133.305 89.39) (end 133.305 111.885) (width 0.2) (layer "B.Cu") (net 8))
 (segment (start 133.305 111.885) (end 137.76 116.34) (width 0.2) (layer "B.Cu") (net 8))
 (segment (start 175.501 92.216) (end 157.435 74.15) (width 0.2) (layer "F.Cu") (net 31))
 (segment (start 175.501 100.559) (end 175.501 92.216) (width 0.2) (layer "F.Cu") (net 31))
 (segment (start 174 102.06) (end 175.501 100.559) (width 0.2) (layer "F.Cu") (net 31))
 (segment (start 151.235039 87.969961) (end 151.235039 122.458) (width 0.2) (layer "B.Cu") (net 35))
 (segment (start 113.999 116.681735) (end 113.999 114.061) (width 0.2) (layer "B.Cu") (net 35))
 (segment (start 138.274039 135.419) (end 132.736265 135.419) (width 0.2) (layer "B.Cu") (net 35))
 (segment (start 113.999 114.061) (end 115.5 112.56) (width 0.2) (layer "B.Cu") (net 35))
 (segment (start 132.736265 135.419) (end 113.999 116.681735) (width 0.2) (layer "B.Cu") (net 35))
 (segment (start 151.235039 122.458) (end 138.274039 135.419) (width 0.2) (layer "B.Cu") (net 35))
 (segment (start 157.435 81.77) (end 151.235039 87.969961) (width 0.2) (layer "B.Cu") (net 35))
 (segment (start 115.5 84) (end 124 92.5) (width 0.2) (layer "F.Cu") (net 33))
 (segment (start 154.325 92.5) (end 157.435 89.39) (width 0.2) (layer "F.Cu") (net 33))
 (segment (start 124 92.5) (end 154.325 92.5) (width 0.2) (layer "F.Cu") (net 33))
 (segment (start 132.121 132.681) (end 115.5 116.06) (width 0.2) (layer "B.Cu") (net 36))
 (segment (start 149.5 87.165) (end 149.5 121.39705) (width 0.2) (layer "B.Cu") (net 36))
 (segment (start 149.5 121.39705) (end 138.21605 132.681) (width 0.2) (layer "B.Cu") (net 36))
 (segment (start 138.21605 132.681) (end 132.121 132.681) (width 0.2) (layer "B.Cu") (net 36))
 (segment (start 157.435 79.23) (end 149.5 87.165) (width 0.2) (layer "B.Cu") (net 36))
 (segment (start 174 98.56) (end 174 93.255) (width 0.2) (layer "F.Cu") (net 32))
 (segment (start 174 93.255) (end 157.435 76.69) (width 0.2) (layer "F.Cu") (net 32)))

